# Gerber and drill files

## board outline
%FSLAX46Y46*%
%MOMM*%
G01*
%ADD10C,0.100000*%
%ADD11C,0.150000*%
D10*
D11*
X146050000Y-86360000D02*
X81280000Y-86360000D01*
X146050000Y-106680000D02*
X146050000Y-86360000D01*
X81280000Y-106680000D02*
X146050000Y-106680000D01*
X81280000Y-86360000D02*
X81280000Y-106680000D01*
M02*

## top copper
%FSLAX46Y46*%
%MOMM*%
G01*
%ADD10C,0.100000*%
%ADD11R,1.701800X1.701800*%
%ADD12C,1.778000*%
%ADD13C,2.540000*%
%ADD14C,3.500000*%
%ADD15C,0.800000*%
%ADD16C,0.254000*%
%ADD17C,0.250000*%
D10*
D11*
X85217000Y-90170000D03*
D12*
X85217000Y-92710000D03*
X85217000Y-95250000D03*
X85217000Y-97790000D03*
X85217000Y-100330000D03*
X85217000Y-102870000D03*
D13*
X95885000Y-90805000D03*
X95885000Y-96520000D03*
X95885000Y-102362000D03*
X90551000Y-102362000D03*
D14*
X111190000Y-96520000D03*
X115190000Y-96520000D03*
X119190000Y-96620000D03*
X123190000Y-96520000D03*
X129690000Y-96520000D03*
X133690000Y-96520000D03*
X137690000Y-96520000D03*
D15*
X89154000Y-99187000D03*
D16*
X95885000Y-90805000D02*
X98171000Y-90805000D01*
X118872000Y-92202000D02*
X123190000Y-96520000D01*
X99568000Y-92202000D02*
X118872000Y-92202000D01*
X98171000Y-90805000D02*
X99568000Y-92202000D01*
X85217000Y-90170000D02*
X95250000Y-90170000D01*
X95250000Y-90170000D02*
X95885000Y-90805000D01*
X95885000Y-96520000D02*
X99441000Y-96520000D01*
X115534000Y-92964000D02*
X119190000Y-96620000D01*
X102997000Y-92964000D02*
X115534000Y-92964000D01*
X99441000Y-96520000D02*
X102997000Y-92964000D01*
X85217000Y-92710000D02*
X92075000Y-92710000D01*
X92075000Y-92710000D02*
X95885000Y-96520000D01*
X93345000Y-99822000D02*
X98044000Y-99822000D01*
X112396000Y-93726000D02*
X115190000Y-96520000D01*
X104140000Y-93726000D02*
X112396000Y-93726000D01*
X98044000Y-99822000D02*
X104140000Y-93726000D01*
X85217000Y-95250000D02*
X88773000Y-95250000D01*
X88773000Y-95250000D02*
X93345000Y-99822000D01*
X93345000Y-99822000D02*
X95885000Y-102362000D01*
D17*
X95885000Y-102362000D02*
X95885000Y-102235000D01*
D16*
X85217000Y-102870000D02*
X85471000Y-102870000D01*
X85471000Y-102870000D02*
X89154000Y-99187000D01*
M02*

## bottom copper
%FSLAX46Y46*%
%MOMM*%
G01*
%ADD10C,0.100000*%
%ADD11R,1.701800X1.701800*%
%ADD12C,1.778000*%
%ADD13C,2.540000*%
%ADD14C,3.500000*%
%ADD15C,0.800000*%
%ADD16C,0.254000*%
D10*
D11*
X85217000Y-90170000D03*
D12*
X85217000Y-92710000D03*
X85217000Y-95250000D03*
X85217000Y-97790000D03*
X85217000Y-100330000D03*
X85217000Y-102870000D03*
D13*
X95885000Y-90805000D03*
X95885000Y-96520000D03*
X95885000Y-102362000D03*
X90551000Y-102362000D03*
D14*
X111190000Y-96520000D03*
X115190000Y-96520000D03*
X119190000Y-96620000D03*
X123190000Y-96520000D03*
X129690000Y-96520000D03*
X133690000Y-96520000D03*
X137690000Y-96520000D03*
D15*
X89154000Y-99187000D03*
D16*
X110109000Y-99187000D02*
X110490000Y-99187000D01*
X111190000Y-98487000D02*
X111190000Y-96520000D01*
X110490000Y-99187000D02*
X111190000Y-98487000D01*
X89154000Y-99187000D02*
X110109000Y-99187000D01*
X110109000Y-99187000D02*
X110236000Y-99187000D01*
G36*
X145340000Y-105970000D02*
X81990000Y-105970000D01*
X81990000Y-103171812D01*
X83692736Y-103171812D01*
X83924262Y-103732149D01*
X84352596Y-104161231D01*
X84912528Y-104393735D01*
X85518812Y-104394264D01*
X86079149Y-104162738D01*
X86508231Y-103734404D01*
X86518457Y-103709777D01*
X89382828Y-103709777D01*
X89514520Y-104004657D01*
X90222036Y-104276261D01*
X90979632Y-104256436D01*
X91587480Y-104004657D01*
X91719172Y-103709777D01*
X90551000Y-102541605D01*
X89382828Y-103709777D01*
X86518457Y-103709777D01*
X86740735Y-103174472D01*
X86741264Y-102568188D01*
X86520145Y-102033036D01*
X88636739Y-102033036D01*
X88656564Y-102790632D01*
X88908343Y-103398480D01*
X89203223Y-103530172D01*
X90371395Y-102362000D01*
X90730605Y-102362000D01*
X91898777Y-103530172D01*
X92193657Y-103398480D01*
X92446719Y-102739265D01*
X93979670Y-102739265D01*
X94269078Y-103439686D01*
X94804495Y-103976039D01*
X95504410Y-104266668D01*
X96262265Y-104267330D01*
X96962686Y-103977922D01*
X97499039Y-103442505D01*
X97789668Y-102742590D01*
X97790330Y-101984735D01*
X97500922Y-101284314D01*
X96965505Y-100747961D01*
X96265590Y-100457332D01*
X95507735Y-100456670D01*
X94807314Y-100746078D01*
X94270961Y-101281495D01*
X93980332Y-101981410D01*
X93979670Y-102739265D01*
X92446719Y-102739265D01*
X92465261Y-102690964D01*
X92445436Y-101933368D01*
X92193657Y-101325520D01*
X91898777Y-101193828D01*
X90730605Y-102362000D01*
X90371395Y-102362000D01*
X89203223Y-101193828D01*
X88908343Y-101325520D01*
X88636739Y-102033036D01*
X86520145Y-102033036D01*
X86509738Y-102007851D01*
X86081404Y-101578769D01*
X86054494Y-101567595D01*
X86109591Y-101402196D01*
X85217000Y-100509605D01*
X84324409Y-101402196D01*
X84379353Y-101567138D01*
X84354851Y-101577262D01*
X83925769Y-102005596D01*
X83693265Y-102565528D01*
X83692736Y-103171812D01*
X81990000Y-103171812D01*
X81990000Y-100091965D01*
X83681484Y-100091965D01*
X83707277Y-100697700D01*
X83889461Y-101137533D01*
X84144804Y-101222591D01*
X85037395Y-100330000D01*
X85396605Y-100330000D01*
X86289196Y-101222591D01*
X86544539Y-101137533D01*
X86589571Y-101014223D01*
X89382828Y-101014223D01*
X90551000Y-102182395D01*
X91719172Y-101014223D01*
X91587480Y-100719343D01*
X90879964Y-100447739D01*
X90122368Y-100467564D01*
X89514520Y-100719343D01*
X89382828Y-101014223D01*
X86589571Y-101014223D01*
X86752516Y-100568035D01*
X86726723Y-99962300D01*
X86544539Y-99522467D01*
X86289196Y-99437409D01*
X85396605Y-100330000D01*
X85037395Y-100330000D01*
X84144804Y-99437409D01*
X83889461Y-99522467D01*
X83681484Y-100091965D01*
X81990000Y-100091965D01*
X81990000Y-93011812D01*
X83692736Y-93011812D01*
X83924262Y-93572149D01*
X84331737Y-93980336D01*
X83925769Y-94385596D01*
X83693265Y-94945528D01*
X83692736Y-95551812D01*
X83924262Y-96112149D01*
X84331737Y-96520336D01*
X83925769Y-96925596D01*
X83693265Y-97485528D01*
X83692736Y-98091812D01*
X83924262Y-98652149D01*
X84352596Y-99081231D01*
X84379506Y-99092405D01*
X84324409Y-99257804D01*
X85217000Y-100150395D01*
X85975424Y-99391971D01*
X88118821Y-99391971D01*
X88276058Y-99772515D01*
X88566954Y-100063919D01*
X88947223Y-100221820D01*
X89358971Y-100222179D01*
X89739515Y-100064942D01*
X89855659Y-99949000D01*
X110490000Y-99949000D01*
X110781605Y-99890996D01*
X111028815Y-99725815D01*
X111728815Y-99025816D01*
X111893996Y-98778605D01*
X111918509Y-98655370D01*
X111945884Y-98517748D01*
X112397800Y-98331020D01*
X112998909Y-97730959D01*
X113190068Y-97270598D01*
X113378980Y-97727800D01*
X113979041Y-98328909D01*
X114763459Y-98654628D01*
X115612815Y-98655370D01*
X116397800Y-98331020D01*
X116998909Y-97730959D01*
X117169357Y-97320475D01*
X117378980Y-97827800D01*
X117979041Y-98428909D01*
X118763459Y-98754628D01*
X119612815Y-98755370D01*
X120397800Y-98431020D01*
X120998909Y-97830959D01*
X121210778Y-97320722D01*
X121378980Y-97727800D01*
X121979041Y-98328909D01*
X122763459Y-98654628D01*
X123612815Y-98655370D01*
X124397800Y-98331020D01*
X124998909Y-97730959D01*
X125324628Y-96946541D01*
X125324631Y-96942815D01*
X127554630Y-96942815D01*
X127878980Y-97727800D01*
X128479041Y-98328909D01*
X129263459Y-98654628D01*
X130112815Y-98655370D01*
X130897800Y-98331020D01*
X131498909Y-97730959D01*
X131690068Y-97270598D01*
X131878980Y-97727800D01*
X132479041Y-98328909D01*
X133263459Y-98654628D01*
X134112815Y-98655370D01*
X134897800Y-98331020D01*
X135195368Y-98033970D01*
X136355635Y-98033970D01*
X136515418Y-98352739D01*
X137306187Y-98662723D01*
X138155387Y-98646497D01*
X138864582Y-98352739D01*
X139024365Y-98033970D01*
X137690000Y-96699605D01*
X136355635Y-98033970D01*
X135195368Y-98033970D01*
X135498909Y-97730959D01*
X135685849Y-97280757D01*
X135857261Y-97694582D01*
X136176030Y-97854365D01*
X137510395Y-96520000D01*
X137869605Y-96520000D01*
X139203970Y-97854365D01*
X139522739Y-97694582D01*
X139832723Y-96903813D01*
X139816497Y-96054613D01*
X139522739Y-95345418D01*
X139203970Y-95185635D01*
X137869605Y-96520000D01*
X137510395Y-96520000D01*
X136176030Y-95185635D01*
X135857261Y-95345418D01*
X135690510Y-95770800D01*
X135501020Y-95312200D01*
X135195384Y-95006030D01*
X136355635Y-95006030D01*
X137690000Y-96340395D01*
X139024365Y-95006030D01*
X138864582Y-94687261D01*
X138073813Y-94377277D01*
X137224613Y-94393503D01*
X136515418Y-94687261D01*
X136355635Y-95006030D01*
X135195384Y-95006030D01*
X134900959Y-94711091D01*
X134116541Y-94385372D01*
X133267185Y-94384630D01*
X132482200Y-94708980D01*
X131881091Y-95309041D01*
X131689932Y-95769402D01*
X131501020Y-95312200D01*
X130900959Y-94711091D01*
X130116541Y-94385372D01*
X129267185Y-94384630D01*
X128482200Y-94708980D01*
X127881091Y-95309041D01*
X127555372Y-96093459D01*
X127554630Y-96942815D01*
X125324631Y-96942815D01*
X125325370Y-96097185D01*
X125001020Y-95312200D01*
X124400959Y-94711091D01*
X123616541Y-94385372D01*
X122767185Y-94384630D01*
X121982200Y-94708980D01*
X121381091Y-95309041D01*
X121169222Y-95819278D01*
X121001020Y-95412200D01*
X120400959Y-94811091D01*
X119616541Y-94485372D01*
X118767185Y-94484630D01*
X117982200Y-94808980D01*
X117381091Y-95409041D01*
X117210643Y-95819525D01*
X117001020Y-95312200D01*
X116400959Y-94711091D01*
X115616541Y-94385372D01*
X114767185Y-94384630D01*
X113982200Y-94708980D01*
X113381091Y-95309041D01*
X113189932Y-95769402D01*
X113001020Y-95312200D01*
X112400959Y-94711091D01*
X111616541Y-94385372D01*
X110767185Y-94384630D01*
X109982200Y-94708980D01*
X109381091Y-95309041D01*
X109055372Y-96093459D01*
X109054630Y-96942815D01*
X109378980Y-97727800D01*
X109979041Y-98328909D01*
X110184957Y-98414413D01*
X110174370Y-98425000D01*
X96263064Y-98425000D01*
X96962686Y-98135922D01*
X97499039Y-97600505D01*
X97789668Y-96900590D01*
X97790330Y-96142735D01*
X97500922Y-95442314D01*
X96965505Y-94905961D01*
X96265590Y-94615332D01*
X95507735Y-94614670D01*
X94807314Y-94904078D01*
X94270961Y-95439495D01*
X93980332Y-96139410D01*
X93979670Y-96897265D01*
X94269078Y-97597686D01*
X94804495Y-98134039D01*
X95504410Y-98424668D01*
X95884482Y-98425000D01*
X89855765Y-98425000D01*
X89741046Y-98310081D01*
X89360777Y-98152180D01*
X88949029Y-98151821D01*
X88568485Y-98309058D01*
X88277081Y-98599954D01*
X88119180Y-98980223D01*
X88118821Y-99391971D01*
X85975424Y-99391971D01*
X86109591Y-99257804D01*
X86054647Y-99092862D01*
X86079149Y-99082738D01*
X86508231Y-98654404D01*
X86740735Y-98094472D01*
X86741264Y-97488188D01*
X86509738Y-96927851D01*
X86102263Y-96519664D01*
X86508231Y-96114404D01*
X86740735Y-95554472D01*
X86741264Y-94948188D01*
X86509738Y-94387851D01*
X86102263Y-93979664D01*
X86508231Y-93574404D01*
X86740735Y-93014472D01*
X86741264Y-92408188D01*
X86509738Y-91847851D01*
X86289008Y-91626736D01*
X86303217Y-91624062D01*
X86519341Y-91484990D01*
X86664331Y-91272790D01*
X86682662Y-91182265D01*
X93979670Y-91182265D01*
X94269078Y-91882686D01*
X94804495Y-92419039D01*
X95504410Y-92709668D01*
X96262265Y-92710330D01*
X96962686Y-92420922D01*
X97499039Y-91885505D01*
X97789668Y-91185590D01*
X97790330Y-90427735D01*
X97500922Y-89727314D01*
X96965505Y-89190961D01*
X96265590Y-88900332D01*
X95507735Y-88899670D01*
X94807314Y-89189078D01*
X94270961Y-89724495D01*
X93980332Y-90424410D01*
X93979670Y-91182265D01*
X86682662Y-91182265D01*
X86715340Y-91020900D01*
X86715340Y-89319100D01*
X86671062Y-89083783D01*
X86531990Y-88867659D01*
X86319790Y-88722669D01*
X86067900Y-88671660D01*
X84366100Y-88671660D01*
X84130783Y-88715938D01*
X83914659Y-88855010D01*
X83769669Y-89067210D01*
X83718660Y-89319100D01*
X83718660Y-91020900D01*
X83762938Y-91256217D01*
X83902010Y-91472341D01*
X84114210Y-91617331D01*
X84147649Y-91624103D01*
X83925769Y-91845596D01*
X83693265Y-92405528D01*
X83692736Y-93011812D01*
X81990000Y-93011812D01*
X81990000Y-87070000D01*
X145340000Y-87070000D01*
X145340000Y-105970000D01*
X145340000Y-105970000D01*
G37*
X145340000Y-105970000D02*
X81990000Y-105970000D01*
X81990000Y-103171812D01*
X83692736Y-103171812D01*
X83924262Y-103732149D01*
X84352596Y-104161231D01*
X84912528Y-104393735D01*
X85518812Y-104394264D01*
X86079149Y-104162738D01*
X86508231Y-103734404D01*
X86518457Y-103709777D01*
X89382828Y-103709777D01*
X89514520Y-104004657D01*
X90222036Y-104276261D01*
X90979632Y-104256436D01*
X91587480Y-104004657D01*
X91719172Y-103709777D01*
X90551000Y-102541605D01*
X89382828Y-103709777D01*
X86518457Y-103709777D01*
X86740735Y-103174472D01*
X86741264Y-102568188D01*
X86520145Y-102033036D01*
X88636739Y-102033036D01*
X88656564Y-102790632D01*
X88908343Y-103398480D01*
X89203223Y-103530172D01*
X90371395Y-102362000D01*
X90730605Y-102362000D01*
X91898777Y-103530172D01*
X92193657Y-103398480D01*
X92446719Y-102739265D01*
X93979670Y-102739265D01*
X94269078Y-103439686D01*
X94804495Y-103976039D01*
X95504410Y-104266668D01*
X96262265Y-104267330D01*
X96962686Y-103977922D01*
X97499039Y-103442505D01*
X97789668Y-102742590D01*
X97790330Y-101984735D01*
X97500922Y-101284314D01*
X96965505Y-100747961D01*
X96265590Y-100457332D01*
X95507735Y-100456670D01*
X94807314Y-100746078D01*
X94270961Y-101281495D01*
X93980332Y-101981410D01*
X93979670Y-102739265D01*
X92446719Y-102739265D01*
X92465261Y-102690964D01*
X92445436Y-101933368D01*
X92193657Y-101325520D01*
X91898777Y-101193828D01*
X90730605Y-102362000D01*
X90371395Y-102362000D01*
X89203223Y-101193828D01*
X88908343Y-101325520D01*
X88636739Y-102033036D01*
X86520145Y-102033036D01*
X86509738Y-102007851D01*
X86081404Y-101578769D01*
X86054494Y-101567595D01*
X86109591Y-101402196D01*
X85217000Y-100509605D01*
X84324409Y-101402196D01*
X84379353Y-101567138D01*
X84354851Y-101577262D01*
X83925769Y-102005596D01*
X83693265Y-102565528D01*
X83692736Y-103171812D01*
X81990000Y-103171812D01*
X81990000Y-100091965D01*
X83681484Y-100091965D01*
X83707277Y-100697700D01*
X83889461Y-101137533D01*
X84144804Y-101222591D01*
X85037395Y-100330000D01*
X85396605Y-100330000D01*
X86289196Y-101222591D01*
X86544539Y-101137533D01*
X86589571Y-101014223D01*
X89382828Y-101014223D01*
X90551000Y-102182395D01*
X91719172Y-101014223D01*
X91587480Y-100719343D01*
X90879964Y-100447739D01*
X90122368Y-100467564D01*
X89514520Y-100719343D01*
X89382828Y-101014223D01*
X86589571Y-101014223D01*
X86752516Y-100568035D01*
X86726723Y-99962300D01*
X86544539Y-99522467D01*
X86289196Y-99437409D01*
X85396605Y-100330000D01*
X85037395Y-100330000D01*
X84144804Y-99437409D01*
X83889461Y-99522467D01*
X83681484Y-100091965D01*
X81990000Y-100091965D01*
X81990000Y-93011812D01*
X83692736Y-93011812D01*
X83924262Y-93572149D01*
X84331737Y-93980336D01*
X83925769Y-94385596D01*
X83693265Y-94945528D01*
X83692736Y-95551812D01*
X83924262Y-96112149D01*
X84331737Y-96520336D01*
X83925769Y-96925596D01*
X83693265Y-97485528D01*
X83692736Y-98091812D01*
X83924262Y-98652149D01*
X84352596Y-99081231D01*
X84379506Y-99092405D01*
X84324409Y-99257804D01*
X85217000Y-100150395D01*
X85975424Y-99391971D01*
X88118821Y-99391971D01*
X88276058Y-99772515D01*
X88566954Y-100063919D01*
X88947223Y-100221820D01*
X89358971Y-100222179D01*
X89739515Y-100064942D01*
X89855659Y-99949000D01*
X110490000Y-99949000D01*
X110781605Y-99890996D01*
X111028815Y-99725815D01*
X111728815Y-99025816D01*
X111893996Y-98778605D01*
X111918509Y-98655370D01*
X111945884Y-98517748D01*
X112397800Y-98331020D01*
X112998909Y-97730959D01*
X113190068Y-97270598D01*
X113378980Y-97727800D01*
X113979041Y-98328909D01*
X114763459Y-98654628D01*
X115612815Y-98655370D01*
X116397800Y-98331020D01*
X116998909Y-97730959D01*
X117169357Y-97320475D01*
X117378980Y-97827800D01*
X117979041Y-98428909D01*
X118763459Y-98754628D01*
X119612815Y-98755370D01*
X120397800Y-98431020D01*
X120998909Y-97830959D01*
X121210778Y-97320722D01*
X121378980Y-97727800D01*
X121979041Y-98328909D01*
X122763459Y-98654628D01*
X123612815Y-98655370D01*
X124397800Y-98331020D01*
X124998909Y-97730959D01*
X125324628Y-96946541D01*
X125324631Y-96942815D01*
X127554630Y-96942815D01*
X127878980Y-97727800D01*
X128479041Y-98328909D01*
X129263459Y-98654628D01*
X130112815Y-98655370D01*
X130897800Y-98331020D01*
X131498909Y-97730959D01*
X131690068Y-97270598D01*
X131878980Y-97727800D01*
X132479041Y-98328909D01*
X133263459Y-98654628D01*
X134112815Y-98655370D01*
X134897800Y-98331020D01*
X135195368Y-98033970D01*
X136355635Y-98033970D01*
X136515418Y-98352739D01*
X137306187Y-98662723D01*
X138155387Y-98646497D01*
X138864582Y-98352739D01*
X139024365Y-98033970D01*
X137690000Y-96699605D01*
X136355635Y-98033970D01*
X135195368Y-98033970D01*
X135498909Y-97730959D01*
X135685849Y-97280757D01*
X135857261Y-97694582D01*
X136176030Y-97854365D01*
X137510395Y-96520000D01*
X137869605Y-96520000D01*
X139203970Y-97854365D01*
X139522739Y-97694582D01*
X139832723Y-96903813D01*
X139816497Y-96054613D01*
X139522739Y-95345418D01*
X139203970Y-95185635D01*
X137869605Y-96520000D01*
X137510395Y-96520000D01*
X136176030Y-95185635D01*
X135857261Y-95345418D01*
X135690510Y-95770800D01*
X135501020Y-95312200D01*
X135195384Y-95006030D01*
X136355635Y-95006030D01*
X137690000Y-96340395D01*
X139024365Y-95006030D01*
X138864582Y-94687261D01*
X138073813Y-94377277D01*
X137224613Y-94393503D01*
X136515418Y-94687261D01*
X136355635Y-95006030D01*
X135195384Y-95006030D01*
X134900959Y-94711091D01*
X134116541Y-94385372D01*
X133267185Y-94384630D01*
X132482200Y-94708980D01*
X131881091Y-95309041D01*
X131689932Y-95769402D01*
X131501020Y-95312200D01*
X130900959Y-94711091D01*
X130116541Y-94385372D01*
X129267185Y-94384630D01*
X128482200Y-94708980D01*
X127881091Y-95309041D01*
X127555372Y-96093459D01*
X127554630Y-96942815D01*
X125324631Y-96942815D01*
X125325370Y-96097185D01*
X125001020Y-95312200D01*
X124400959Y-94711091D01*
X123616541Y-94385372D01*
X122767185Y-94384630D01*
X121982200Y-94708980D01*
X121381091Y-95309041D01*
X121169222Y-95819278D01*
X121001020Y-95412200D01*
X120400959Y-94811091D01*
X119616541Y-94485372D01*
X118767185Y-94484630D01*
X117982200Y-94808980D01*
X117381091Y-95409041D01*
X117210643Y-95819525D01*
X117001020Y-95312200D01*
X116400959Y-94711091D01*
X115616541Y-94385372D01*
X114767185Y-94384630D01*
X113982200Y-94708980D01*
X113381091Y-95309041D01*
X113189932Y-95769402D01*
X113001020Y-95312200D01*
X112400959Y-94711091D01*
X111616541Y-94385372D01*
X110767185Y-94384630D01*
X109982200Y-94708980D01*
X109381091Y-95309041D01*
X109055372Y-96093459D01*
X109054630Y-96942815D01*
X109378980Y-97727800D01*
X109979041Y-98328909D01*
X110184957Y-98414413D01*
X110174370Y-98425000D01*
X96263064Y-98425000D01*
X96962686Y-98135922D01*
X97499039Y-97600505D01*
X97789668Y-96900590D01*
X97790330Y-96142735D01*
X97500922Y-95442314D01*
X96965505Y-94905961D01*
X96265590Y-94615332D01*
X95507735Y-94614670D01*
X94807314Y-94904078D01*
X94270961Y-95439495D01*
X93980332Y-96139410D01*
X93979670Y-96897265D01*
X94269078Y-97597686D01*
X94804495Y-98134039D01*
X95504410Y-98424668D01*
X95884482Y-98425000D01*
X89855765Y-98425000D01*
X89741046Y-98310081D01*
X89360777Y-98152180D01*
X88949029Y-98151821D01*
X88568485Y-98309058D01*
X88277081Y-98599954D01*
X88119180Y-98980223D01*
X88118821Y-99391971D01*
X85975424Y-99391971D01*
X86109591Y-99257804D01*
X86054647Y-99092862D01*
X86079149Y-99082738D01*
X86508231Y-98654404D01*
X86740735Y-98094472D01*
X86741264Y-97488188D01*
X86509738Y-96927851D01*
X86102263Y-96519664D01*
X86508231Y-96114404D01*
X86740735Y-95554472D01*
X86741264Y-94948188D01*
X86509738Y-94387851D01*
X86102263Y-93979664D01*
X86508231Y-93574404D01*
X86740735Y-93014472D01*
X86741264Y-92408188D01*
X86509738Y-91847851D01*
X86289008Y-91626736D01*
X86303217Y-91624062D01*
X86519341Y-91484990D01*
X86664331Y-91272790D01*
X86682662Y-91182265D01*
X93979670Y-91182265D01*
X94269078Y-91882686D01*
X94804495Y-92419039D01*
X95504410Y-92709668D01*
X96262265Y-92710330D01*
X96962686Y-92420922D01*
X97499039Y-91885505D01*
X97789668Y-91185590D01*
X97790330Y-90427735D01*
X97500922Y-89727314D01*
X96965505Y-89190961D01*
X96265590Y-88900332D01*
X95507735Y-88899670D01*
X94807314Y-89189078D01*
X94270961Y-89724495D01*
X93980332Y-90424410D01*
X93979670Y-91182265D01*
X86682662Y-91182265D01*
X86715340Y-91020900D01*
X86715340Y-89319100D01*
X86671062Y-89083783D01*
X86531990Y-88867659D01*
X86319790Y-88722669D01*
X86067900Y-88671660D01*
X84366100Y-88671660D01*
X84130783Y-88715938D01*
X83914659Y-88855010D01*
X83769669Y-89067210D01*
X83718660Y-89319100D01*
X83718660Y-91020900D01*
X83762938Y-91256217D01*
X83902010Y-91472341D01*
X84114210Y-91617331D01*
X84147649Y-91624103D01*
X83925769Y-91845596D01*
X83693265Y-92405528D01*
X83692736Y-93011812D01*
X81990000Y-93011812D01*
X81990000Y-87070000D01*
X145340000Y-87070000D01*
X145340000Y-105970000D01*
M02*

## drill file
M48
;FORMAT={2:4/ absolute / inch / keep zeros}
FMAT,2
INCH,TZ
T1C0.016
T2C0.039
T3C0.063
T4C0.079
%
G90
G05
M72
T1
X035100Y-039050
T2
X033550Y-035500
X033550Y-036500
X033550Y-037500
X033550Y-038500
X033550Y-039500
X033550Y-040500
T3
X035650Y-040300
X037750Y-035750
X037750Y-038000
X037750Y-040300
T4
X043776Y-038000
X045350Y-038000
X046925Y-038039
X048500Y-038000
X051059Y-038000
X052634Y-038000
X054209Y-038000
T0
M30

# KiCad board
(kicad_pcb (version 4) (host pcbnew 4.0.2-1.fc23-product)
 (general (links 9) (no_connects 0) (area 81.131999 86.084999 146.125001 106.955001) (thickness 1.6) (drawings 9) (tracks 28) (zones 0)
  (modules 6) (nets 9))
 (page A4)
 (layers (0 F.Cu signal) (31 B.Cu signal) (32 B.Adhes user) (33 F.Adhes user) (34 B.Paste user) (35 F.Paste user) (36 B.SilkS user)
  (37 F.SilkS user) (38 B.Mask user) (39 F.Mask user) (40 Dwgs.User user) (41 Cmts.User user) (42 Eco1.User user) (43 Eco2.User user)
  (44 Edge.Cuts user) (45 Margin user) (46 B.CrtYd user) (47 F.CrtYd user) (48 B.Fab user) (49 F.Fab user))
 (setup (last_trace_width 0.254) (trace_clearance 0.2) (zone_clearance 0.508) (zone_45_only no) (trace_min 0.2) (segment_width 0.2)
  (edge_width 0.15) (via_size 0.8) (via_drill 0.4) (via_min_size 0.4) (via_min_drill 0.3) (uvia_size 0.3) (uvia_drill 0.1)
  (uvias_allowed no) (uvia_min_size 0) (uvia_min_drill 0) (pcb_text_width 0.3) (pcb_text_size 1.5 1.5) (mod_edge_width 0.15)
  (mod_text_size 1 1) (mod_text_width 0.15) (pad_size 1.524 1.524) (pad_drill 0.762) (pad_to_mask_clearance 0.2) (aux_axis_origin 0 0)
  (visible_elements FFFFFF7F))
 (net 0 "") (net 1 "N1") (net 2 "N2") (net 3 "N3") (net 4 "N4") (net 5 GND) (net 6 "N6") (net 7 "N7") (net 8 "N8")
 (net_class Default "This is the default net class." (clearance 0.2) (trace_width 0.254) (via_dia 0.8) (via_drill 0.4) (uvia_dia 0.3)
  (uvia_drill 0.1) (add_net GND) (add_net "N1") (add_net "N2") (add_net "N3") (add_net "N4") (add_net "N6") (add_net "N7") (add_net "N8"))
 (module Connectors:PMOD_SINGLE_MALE (layer F.Cu) (at 83.185 96.52 90)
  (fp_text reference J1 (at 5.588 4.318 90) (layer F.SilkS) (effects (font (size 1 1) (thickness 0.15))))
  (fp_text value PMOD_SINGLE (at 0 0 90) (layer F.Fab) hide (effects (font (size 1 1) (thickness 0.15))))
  (pad 1 thru_hole rect (at 6.35 2.032 270) (size 1.7018 1.7018) (drill 0.9906) (layers *.Cu *.Mask F.SilkS) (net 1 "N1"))
  (pad 2 thru_hole circle (at 3.81 2.032 270) (size 1.778 1.778) (drill 0.9906) (layers *.Cu *.Mask F.SilkS) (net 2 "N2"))
  (pad 3 thru_hole circle (at 1.27 2.032 270) (size 1.778 1.778) (drill 0.9906) (layers *.Cu *.Mask F.SilkS) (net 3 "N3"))
  (pad 4 thru_hole circle (at -1.27 2.032 270) (size 1.778 1.778) (drill 0.9906) (layers *.Cu *.Mask F.SilkS) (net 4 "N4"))
  (pad 5 thru_hole circle (at -3.81 2.032 270) (size 1.778 1.778) (drill 0.9906) (layers *.Cu *.Mask F.SilkS) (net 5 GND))
  (pad 6 thru_hole circle (at -6.35 2.032 270) (size 1.778 1.778) (drill 0.9906) (layers *.Cu *.Mask F.SilkS) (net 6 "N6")))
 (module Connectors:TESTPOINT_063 (layer F.Cu) (at 95.885 90.805)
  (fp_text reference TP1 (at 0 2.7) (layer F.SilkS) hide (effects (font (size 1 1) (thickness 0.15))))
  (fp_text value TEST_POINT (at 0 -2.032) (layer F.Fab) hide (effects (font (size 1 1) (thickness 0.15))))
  (pad 1 thru_hole circle (at 0 0) (size 2.54 2.54) (drill 1.6002) (layers *.Cu *.Mask F.SilkS) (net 1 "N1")))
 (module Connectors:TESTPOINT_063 (layer F.Cu) (at 95.885 96.52)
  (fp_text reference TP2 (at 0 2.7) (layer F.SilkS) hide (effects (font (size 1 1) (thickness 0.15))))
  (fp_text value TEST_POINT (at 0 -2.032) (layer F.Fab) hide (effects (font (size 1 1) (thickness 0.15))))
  (pad 1 thru_hole circle (at 0 0) (size 2.54 2.54) (drill 1.6002) (layers *.Cu *.Mask F.SilkS) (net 2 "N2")))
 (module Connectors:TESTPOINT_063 (layer F.Cu) (at 95.885 102.362)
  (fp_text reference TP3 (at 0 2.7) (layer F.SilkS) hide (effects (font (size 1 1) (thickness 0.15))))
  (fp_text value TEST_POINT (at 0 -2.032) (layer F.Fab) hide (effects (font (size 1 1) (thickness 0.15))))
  (pad 1 thru_hole circle (at 0 0) (size 2.54 2.54) (drill 1.6002) (layers *.Cu *.Mask F.SilkS) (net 3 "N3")))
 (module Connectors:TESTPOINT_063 (layer F.Cu) (at 90.551 102.362)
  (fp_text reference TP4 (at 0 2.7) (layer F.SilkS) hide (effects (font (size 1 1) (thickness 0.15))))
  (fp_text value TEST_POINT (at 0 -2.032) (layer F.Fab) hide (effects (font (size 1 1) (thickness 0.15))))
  (pad 1 thru_hole circle (at 0 0) (size 2.54 2.54) (drill 1.6002) (layers *.Cu *.Mask F.SilkS) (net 5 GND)))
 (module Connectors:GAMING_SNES (layer F.Cu) (at 123.19 96.52)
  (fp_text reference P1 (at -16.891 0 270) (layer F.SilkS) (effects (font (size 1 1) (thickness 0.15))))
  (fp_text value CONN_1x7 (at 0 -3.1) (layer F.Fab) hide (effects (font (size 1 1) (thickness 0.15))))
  (pad 1 thru_hole circle (at -12 0) (size 3.5 3.5) (drill 2) (layers *.Cu *.Mask F.SilkS) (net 6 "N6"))
  (pad 2 thru_hole circle (at -8 0) (size 3.5 3.5) (drill 2) (layers *.Cu *.Mask F.SilkS) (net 3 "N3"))
  (pad 3 thru_hole circle (at -4 0.1) (size 3.5 3.5) (drill 2) (layers *.Cu *.Mask F.SilkS) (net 2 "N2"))
  (pad 4 thru_hole circle (at 0 0) (size 3.5 3.5) (drill 2) (layers *.Cu *.Mask F.SilkS) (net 1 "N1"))
  (pad 5 thru_hole circle (at 6.5 0) (size 3.5 3.5) (drill 2) (layers *.Cu *.Mask F.SilkS) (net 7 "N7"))
  (pad 6 thru_hole circle (at 10.5 0) (size 3.5 3.5) (drill 2) (layers *.Cu *.Mask F.SilkS) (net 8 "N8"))
  (pad 7 thru_hole circle (at 14.5 0) (size 3.5 3.5) (drill 2) (layers *.Cu *.Mask F.SilkS) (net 5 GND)))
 (gr_line (start 146.05 86.36) (end 81.28 86.36) (angle 90) (layer Edge.Cuts) (width 0.15))
 (gr_line (start 146.05 106.68) (end 146.05 86.36) (angle 90) (layer Edge.Cuts) (width 0.15))
 (gr_line (start 81.28 106.68) (end 146.05 106.68) (angle 90) (layer Edge.Cuts) (width 0.15))
 (gr_line (start 81.28 86.36) (end 81.28 106.68) (angle 90) (layer Edge.Cuts) (width 0.15))
 (segment (start 95.885 90.805) (end 98.171 90.805) (width 0.254) (layer F.Cu) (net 1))
 (segment (start 118.872 92.202) (end 123.19 96.52) (width 0.254) (layer F.Cu) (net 1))
 (segment (start 99.568 92.202) (end 118.872 92.202) (width 0.254) (layer F.Cu) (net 1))
 (segment (start 98.171 90.805) (end 99.568 92.202) (width 0.254) (layer F.Cu) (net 1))
 (segment (start 85.217 90.17) (end 95.25 90.17) (width 0.254) (layer F.Cu) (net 1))
 (segment (start 95.25 90.17) (end 95.885 90.805) (width 0.254) (layer F.Cu) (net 1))
 (segment (start 95.885 96.52) (end 99.441 96.52) (width 0.254) (layer F.Cu) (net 2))
 (segment (start 115.534 92.964) (end 119.19 96.62) (width 0.254) (layer F.Cu) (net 2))
 (segment (start 102.997 92.964) (end 115.534 92.964) (width 0.254) (layer F.Cu) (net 2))
 (segment (start 99.441 96.52) (end 102.997 92.964) (width 0.254) (layer F.Cu) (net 2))
 (segment (start 85.217 92.71) (end 92.075 92.71) (width 0.254) (layer F.Cu) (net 2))
 (segment (start 92.075 92.71) (end 95.885 96.52) (width 0.254) (layer F.Cu) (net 2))
 (segment (start 93.345 99.822) (end 98.044 99.822) (width 0.254) (layer F.Cu) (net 3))
 (segment (start 112.396 93.726) (end 115.19 96.52) (width 0.254) (layer F.Cu) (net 3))
 (segment (start 104.14 93.726) (end 112.396 93.726) (width 0.254) (layer F.Cu) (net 3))
 (segment (start 98.044 99.822) (end 104.14 93.726) (width 0.254) (layer F.Cu) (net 3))
 (segment (start 85.217 95.25) (end 88.773 95.25) (width 0.254) (layer F.Cu) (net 3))
 (segment (start 88.773 95.25) (end 93.345 99.822) (width 0.254) (layer F.Cu) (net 3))
 (segment (start 93.345 99.822) (end 95.885 102.362) (width 0.254) (layer F.Cu) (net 3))
 (segment (start 95.885 102.362) (end 95.885 102.235) (width 0.25) (layer F.Cu) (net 3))
 (segment (start 110.109 99.187) (end 110.49 99.187) (width 0.254) (layer B.Cu) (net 6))
 (segment (start 111.19 98.487) (end 111.19 96.52) (width 0.254) (layer B.Cu) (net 6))
 (segment (start 110.49 99.187) (end 111.19 98.487) (width 0.254) (layer B.Cu) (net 6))
 (segment (start 85.217 102.87) (end 85.471 102.87) (width 0.254) (layer F.Cu) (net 6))
 (segment (start 85.471 102.87) (end 89.154 99.187) (width 0.254) (layer F.Cu) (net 6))
 (via (at 89.154 99.187) (size 0.8) (drill 0.4) (layers F.Cu B.Cu) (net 6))
 (segment (start 89.154 99.187) (end 110.109 99.187) (width 0.254) (layer B.Cu) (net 6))
 (segment (start 110.109 99.187) (end 110.236 99.187) (width 0.254) (layer B.Cu) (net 6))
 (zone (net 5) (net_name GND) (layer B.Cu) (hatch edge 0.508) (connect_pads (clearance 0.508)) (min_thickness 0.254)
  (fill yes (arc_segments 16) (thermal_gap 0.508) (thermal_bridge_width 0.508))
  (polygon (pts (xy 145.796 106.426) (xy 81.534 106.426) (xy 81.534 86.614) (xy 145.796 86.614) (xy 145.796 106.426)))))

